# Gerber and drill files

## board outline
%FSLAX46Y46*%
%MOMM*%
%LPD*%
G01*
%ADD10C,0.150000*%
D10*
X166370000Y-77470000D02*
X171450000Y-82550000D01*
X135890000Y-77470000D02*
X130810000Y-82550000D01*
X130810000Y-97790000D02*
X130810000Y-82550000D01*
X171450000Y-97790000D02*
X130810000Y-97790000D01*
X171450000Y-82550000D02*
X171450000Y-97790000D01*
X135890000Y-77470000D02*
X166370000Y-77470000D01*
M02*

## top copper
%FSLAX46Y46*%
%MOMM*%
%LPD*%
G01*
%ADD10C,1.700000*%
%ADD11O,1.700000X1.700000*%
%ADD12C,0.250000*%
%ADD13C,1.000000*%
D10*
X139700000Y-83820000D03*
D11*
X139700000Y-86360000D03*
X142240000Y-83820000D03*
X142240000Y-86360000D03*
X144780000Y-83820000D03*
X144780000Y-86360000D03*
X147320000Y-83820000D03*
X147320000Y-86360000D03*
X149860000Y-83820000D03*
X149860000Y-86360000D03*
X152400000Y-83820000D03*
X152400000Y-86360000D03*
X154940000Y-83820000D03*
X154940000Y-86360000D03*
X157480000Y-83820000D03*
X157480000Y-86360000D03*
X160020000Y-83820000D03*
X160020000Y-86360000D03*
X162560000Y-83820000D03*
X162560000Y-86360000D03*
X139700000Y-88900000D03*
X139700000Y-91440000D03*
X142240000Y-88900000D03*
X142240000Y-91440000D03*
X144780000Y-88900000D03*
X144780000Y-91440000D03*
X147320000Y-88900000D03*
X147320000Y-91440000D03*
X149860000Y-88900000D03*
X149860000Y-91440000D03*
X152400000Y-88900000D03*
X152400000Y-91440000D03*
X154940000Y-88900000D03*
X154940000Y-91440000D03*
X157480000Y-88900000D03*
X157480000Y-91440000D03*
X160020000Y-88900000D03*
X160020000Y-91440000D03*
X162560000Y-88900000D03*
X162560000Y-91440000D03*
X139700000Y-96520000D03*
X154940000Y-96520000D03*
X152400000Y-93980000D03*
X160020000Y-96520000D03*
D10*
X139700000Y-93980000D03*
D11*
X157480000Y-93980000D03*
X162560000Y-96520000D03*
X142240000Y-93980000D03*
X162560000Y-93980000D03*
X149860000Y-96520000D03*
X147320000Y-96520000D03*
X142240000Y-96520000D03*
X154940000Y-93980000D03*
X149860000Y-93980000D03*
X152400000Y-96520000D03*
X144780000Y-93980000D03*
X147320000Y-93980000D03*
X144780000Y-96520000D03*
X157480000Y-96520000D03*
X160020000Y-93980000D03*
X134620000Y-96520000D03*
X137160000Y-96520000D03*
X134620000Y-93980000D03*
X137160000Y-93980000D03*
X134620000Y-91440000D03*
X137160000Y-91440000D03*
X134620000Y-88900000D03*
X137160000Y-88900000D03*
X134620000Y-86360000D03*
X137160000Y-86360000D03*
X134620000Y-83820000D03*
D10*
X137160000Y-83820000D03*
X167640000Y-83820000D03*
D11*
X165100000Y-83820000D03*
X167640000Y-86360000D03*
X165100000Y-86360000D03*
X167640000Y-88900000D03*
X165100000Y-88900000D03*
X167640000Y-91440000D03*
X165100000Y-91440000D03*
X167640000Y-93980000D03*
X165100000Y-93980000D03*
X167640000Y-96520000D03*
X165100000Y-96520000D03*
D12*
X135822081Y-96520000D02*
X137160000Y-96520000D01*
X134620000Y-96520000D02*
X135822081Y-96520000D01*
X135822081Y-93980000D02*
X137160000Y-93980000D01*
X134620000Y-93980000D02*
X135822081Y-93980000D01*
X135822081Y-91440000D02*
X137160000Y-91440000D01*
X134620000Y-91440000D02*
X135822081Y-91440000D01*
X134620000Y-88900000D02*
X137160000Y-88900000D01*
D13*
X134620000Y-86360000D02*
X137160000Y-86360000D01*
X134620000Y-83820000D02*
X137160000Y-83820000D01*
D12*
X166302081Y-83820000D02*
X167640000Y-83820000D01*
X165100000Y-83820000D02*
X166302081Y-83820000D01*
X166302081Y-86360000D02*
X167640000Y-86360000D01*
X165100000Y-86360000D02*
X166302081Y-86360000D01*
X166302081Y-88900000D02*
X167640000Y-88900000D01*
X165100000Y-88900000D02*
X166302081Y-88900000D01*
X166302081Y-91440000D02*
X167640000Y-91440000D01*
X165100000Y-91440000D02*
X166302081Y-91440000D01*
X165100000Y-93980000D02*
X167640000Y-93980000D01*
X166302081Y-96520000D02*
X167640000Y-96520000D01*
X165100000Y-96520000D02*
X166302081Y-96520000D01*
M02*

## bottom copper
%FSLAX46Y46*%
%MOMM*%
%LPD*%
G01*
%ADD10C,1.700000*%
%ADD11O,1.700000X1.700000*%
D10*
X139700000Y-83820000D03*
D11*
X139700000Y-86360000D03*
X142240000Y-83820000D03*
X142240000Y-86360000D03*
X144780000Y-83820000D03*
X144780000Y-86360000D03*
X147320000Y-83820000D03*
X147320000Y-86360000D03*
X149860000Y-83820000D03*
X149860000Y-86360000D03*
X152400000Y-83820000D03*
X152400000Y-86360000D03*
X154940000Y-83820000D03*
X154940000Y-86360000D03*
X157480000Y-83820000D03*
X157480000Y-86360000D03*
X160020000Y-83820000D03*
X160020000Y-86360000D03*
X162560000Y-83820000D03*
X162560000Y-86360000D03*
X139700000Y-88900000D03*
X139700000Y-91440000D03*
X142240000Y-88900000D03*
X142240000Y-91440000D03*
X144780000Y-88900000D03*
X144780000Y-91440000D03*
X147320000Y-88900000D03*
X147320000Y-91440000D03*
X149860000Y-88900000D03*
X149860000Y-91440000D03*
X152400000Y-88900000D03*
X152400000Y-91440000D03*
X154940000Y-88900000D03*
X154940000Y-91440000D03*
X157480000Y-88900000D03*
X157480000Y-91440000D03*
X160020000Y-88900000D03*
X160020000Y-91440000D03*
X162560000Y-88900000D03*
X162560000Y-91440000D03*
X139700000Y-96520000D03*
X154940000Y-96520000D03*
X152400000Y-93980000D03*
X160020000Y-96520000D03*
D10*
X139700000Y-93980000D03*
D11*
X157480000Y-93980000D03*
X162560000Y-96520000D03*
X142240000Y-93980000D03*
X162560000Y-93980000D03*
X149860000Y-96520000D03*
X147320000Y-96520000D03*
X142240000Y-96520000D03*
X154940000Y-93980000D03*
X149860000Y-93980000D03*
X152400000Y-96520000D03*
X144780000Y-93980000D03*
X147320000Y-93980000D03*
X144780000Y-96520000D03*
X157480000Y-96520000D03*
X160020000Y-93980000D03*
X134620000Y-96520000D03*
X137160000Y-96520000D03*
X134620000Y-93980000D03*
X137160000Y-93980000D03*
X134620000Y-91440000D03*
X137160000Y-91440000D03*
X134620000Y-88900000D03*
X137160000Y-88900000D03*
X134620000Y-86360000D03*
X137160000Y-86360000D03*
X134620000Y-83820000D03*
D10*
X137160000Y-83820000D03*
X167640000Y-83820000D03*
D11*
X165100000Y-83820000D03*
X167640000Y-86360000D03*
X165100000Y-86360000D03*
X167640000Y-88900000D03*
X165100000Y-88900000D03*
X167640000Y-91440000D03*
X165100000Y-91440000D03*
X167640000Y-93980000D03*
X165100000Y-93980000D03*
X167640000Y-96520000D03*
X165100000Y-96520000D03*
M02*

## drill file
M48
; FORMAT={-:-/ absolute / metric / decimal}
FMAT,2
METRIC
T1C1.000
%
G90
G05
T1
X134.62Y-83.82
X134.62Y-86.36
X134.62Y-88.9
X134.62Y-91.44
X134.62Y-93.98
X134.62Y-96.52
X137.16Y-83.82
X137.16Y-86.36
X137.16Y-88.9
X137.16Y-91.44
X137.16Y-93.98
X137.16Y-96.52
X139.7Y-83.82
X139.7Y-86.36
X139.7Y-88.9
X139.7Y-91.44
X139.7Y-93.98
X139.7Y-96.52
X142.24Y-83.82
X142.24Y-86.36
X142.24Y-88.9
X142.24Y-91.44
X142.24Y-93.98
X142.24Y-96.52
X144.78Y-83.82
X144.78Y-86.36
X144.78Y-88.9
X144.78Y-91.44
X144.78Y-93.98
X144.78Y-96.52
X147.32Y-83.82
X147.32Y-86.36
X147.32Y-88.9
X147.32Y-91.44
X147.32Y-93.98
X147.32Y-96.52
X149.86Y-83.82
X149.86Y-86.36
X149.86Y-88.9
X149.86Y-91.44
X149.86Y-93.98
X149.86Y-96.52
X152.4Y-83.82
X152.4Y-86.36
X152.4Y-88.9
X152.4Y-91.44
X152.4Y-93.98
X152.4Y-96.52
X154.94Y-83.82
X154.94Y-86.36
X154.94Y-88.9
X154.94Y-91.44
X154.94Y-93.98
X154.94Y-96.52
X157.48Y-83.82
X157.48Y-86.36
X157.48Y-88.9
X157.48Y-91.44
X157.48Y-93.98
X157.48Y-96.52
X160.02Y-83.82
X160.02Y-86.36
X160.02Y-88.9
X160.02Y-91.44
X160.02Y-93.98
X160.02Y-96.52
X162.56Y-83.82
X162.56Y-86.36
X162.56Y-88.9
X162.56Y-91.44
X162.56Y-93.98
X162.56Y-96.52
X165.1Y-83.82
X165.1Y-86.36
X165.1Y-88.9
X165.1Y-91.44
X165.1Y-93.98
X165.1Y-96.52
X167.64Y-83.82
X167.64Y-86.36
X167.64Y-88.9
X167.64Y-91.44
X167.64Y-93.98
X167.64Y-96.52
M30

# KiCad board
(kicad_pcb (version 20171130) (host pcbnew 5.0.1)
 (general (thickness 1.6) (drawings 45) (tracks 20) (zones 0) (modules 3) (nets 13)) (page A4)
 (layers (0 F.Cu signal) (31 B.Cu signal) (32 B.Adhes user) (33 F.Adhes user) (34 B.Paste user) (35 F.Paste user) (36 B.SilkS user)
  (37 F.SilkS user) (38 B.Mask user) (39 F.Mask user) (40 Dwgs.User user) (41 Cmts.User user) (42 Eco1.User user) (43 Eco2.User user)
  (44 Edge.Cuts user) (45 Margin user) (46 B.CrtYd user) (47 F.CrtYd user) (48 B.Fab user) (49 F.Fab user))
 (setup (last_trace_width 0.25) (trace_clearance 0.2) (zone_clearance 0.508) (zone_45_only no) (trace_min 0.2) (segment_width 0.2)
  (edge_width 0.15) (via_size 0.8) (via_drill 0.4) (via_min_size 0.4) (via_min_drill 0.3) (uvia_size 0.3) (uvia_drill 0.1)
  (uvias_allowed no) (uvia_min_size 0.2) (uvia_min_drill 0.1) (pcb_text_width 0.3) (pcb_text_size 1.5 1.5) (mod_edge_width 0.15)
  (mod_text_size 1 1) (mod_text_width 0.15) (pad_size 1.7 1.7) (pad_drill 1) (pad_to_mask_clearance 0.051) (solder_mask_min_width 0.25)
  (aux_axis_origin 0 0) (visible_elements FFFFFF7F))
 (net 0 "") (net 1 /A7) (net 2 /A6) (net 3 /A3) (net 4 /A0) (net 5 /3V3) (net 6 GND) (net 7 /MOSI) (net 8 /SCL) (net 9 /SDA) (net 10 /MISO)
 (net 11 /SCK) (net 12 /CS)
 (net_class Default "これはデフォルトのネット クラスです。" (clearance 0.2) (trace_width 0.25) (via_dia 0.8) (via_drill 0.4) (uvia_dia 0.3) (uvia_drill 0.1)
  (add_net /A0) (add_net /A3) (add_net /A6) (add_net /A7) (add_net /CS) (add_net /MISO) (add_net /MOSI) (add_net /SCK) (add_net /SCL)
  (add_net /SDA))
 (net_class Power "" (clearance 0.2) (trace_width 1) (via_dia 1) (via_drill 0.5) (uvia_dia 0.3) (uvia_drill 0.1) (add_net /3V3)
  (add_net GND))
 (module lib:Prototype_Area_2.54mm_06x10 (layer F.Cu) (at 139.7 83.82 90)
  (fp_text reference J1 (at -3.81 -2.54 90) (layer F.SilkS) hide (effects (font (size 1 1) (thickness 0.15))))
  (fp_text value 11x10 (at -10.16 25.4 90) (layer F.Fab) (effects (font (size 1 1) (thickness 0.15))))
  (pad 1 thru_hole circle (at 0 0 90) (size 1.7 1.7) (drill 1) (layers *.Cu *.Mask))
  (pad 2 thru_hole oval (at -2.54 0 90) (size 1.7 1.7) (drill 1) (layers *.Cu *.Mask))
  (pad 7 thru_hole oval (at 0 2.54 90) (size 1.7 1.7) (drill 1) (layers *.Cu *.Mask))
  (pad 8 thru_hole oval (at -2.54 2.54 90) (size 1.7 1.7) (drill 1) (layers *.Cu *.Mask))
  (pad 13 thru_hole oval (at 0 5.08 90) (size 1.7 1.7) (drill 1) (layers *.Cu *.Mask))
  (pad 14 thru_hole oval (at -2.54 5.08 90) (size 1.7 1.7) (drill 1) (layers *.Cu *.Mask))
  (pad 19 thru_hole oval (at 0 7.62 90) (size 1.7 1.7) (drill 1) (layers *.Cu *.Mask))
  (pad 20 thru_hole oval (at -2.54 7.62 90) (size 1.7 1.7) (drill 1) (layers *.Cu *.Mask))
  (pad 25 thru_hole oval (at 0 10.16 90) (size 1.7 1.7) (drill 1) (layers *.Cu *.Mask))
  (pad 26 thru_hole oval (at -2.54 10.16 90) (size 1.7 1.7) (drill 1) (layers *.Cu *.Mask))
  (pad 31 thru_hole oval (at 0 12.7 90) (size 1.7 1.7) (drill 1) (layers *.Cu *.Mask))
  (pad 32 thru_hole oval (at -2.54 12.7 90) (size 1.7 1.7) (drill 1) (layers *.Cu *.Mask))
  (pad 37 thru_hole oval (at 0 15.24 90) (size 1.7 1.7) (drill 1) (layers *.Cu *.Mask))
  (pad 38 thru_hole oval (at -2.54 15.24 90) (size 1.7 1.7) (drill 1) (layers *.Cu *.Mask))
  (pad 43 thru_hole oval (at 0 17.78 90) (size 1.7 1.7) (drill 1) (layers *.Cu *.Mask))
  (pad 44 thru_hole oval (at -2.54 17.78 90) (size 1.7 1.7) (drill 1) (layers *.Cu *.Mask))
  (pad 49 thru_hole oval (at 0 20.32 90) (size 1.7 1.7) (drill 1) (layers *.Cu *.Mask))
  (pad 50 thru_hole oval (at -2.54 20.32 90) (size 1.7 1.7) (drill 1) (layers *.Cu *.Mask))
  (pad 55 thru_hole oval (at 0 22.86 90) (size 1.7 1.7) (drill 1) (layers *.Cu *.Mask))
  (pad 56 thru_hole oval (at -2.54 22.86 90) (size 1.7 1.7) (drill 1) (layers *.Cu *.Mask))
  (pad 3 thru_hole oval (at -5.08 0 90) (size 1.7 1.7) (drill 1) (layers *.Cu *.Mask))
  (pad 4 thru_hole oval (at -7.62 0 90) (size 1.7 1.7) (drill 1) (layers *.Cu *.Mask))
  (pad 9 thru_hole oval (at -5.08 2.54 90) (size 1.7 1.7) (drill 1) (layers *.Cu *.Mask))
  (pad 10 thru_hole oval (at -7.62 2.54 90) (size 1.7 1.7) (drill 1) (layers *.Cu *.Mask))
  (pad 15 thru_hole oval (at -5.08 5.08 90) (size 1.7 1.7) (drill 1) (layers *.Cu *.Mask))
  (pad 16 thru_hole oval (at -7.62 5.08 90) (size 1.7 1.7) (drill 1) (layers *.Cu *.Mask))
  (pad 21 thru_hole oval (at -5.08 7.62 90) (size 1.7 1.7) (drill 1) (layers *.Cu *.Mask))
  (pad 22 thru_hole oval (at -7.62 7.62 90) (size 1.7 1.7) (drill 1) (layers *.Cu *.Mask))
  (pad 27 thru_hole oval (at -5.08 10.16 90) (size 1.7 1.7) (drill 1) (layers *.Cu *.Mask))
  (pad 28 thru_hole oval (at -7.62 10.16 90) (size 1.7 1.7) (drill 1) (layers *.Cu *.Mask))
  (pad 33 thru_hole oval (at -5.08 12.7 90) (size 1.7 1.7) (drill 1) (layers *.Cu *.Mask))
  (pad 34 thru_hole oval (at -7.62 12.7 90) (size 1.7 1.7) (drill 1) (layers *.Cu *.Mask))
  (pad 39 thru_hole oval (at -5.08 15.24 90) (size 1.7 1.7) (drill 1) (layers *.Cu *.Mask))
  (pad 40 thru_hole oval (at -7.62 15.24 90) (size 1.7 1.7) (drill 1) (layers *.Cu *.Mask))
  (pad 45 thru_hole oval (at -5.08 17.78 90) (size 1.7 1.7) (drill 1) (layers *.Cu *.Mask))
  (pad 46 thru_hole oval (at -7.62 17.78 90) (size 1.7 1.7) (drill 1) (layers *.Cu *.Mask))
  (pad 51 thru_hole oval (at -5.08 20.32 90) (size 1.7 1.7) (drill 1) (layers *.Cu *.Mask))
  (pad 52 thru_hole oval (at -7.62 20.32 90) (size 1.7 1.7) (drill 1) (layers *.Cu *.Mask))
  (pad 57 thru_hole oval (at -5.08 22.86 90) (size 1.7 1.7) (drill 1) (layers *.Cu *.Mask))
  (pad 58 thru_hole oval (at -7.62 22.86 90) (size 1.7 1.7) (drill 1) (layers *.Cu *.Mask))
  (pad 6 thru_hole oval (at -12.7 0 90) (size 1.7 1.7) (drill 1) (layers *.Cu *.Mask))
  (pad 42 thru_hole oval (at -12.7 15.24 90) (size 1.7 1.7) (drill 1) (layers *.Cu *.Mask))
  (pad 35 thru_hole oval (at -10.16 12.7 90) (size 1.7 1.7) (drill 1) (layers *.Cu *.Mask))
  (pad 54 thru_hole oval (at -12.7 20.32 90) (size 1.7 1.7) (drill 1) (layers *.Cu *.Mask))
  (pad 5 thru_hole circle (at -10.16 0 90) (size 1.7 1.7) (drill 1) (layers *.Cu *.Mask))
  (pad 47 thru_hole oval (at -10.16 17.78 90) (size 1.7 1.7) (drill 1) (layers *.Cu *.Mask))
  (pad 60 thru_hole oval (at -12.7 22.86 90) (size 1.7 1.7) (drill 1) (layers *.Cu *.Mask))
  (pad 11 thru_hole oval (at -10.16 2.54 90) (size 1.7 1.7) (drill 1) (layers *.Cu *.Mask))
  (pad 59 thru_hole oval (at -10.16 22.86 90) (size 1.7 1.7) (drill 1) (layers *.Cu *.Mask))
  (pad 30 thru_hole oval (at -12.7 10.16 90) (size 1.7 1.7) (drill 1) (layers *.Cu *.Mask))
  (pad 24 thru_hole oval (at -12.7 7.62 90) (size 1.7 1.7) (drill 1) (layers *.Cu *.Mask))
  (pad 12 thru_hole oval (at -12.7 2.54 90) (size 1.7 1.7) (drill 1) (layers *.Cu *.Mask))
  (pad 41 thru_hole oval (at -10.16 15.24 90) (size 1.7 1.7) (drill 1) (layers *.Cu *.Mask))
  (pad 29 thru_hole oval (at -10.16 10.16 90) (size 1.7 1.7) (drill 1) (layers *.Cu *.Mask))
  (pad 36 thru_hole oval (at -12.7 12.7 90) (size 1.7 1.7) (drill 1) (layers *.Cu *.Mask))
  (pad 17 thru_hole oval (at -10.16 5.08 90) (size 1.7 1.7) (drill 1) (layers *.Cu *.Mask))
  (pad 23 thru_hole oval (at -10.16 7.62 90) (size 1.7 1.7) (drill 1) (layers *.Cu *.Mask))
  (pad 18 thru_hole oval (at -12.7 5.08 90) (size 1.7 1.7) (drill 1) (layers *.Cu *.Mask))
  (pad 48 thru_hole oval (at -12.7 17.78 90) (size 1.7 1.7) (drill 1) (layers *.Cu *.Mask))
  (pad 53 thru_hole oval (at -10.16 20.32 90) (size 1.7 1.7) (drill 1) (layers *.Cu *.Mask)))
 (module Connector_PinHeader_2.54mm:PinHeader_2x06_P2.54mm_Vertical (layer B.Cu) (at 137.16 83.82 180)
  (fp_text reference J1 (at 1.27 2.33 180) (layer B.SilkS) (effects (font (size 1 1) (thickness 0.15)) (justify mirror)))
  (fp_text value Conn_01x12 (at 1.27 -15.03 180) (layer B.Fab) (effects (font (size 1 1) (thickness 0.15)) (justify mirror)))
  (pad 12 thru_hole oval (at 2.54 -12.7 180) (size 1.7 1.7) (drill 1) (layers *.Cu *.Mask) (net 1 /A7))
  (pad 11 thru_hole oval (at 0 -12.7 180) (size 1.7 1.7) (drill 1) (layers *.Cu *.Mask) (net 1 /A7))
  (pad 10 thru_hole oval (at 2.54 -10.16 180) (size 1.7 1.7) (drill 1) (layers *.Cu *.Mask) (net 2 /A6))
  (pad 9 thru_hole oval (at 0 -10.16 180) (size 1.7 1.7) (drill 1) (layers *.Cu *.Mask) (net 2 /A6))
  (pad 8 thru_hole oval (at 2.54 -7.62 180) (size 1.7 1.7) (drill 1) (layers *.Cu *.Mask) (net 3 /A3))
  (pad 7 thru_hole oval (at 0 -7.62 180) (size 1.7 1.7) (drill 1) (layers *.Cu *.Mask) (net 3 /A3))
  (pad 6 thru_hole oval (at 2.54 -5.08 180) (size 1.7 1.7) (drill 1) (layers *.Cu *.Mask) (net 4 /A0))
  (pad 5 thru_hole oval (at 0 -5.08 180) (size 1.7 1.7) (drill 1) (layers *.Cu *.Mask) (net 4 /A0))
  (pad 4 thru_hole oval (at 2.54 -2.54 180) (size 1.7 1.7) (drill 1) (layers *.Cu *.Mask) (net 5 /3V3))
  (pad 3 thru_hole oval (at 0 -2.54 180) (size 1.7 1.7) (drill 1) (layers *.Cu *.Mask) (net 5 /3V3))
  (pad 2 thru_hole oval (at 2.54 0 180) (size 1.7 1.7) (drill 1) (layers *.Cu *.Mask) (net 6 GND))
  (pad 1 thru_hole circle (at 0 0 180) (size 1.7 1.7) (drill 1) (layers *.Cu *.Mask) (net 6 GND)))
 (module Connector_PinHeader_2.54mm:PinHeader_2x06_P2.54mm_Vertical (layer B.Cu) (at 167.64 83.82 180)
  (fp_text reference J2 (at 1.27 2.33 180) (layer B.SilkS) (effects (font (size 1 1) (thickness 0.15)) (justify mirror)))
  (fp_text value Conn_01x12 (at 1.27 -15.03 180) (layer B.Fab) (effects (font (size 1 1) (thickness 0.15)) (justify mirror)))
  (pad 1 thru_hole circle (at 0 0 180) (size 1.7 1.7) (drill 1) (layers *.Cu *.Mask) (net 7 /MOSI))
  (pad 2 thru_hole oval (at 2.54 0 180) (size 1.7 1.7) (drill 1) (layers *.Cu *.Mask) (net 7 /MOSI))
  (pad 3 thru_hole oval (at 0 -2.54 180) (size 1.7 1.7) (drill 1) (layers *.Cu *.Mask) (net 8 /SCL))
  (pad 4 thru_hole oval (at 2.54 -2.54 180) (size 1.7 1.7) (drill 1) (layers *.Cu *.Mask) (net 8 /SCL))
  (pad 5 thru_hole oval (at 0 -5.08 180) (size 1.7 1.7) (drill 1) (layers *.Cu *.Mask) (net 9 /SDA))
  (pad 6 thru_hole oval (at 2.54 -5.08 180) (size 1.7 1.7) (drill 1) (layers *.Cu *.Mask) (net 9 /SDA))
  (pad 7 thru_hole oval (at 0 -7.62 180) (size 1.7 1.7) (drill 1) (layers *.Cu *.Mask) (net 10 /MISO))
  (pad 8 thru_hole oval (at 2.54 -7.62 180) (size 1.7 1.7) (drill 1) (layers *.Cu *.Mask) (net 10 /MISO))
  (pad 9 thru_hole oval (at 0 -10.16 180) (size 1.7 1.7) (drill 1) (layers *.Cu *.Mask) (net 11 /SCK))
  (pad 10 thru_hole oval (at 2.54 -10.16 180) (size 1.7 1.7) (drill 1) (layers *.Cu *.Mask) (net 11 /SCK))
  (pad 11 thru_hole oval (at 0 -12.7 180) (size 1.7 1.7) (drill 1) (layers *.Cu *.Mask) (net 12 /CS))
  (pad 12 thru_hole oval (at 2.54 -12.7 180) (size 1.7 1.7) (drill 1) (layers *.Cu *.Mask) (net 12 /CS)))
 (gr_line (start 166.37 77.47) (end 171.45 82.55) (layer Edge.Cuts) (width 0.15))
 (gr_line (start 135.89 77.47) (end 130.81 82.55) (layer Edge.Cuts) (width 0.15))
 (gr_line (start 130.81 97.79) (end 130.81 82.55) (layer Edge.Cuts) (width 0.15))
 (gr_line (start 171.45 97.79) (end 130.81 97.79) (layer Edge.Cuts) (width 0.15))
 (gr_line (start 171.45 82.55) (end 171.45 97.79) (layer Edge.Cuts) (width 0.15))
 (gr_line (start 135.89 77.47) (end 166.37 77.47) (layer Edge.Cuts) (width 0.15))
 (segment (start 135.822081 96.52) (end 137.16 96.52) (width 0.25) (layer F.Cu) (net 1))
 (segment (start 134.62 96.52) (end 135.822081 96.52) (width 0.25) (layer F.Cu) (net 1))
 (segment (start 135.822081 93.98) (end 137.16 93.98) (width 0.25) (layer F.Cu) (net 2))
 (segment (start 134.62 93.98) (end 135.822081 93.98) (width 0.25) (layer F.Cu) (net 2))
 (segment (start 135.822081 91.44) (end 137.16 91.44) (width 0.25) (layer F.Cu) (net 3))
 (segment (start 134.62 91.44) (end 135.822081 91.44) (width 0.25) (layer F.Cu) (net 3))
 (segment (start 134.62 88.9) (end 137.16 88.9) (width 0.25) (layer F.Cu) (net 4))
 (segment (start 134.62 86.36) (end 137.16 86.36) (width 1) (layer F.Cu) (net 5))
 (segment (start 134.62 83.82) (end 137.16 83.82) (width 1) (layer F.Cu) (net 6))
 (segment (start 166.302081 83.82) (end 167.64 83.82) (width 0.25) (layer F.Cu) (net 7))
 (segment (start 165.1 83.82) (end 166.302081 83.82) (width 0.25) (layer F.Cu) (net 7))
 (segment (start 166.302081 86.36) (end 167.64 86.36) (width 0.25) (layer F.Cu) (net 8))
 (segment (start 165.1 86.36) (end 166.302081 86.36) (width 0.25) (layer F.Cu) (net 8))
 (segment (start 166.302081 88.9) (end 167.64 88.9) (width 0.25) (layer F.Cu) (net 9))
 (segment (start 165.1 88.9) (end 166.302081 88.9) (width 0.25) (layer F.Cu) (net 9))
 (segment (start 166.302081 91.44) (end 167.64 91.44) (width 0.25) (layer F.Cu) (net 10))
 (segment (start 165.1 91.44) (end 166.302081 91.44) (width 0.25) (layer F.Cu) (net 10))
 (segment (start 165.1 93.98) (end 167.64 93.98) (width 0.25) (layer F.Cu) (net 11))
 (segment (start 166.302081 96.52) (end 167.64 96.52) (width 0.25) (layer F.Cu) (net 12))
 (segment (start 165.1 96.52) (end 166.302081 96.52) (width 0.25) (layer F.Cu) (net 12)))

